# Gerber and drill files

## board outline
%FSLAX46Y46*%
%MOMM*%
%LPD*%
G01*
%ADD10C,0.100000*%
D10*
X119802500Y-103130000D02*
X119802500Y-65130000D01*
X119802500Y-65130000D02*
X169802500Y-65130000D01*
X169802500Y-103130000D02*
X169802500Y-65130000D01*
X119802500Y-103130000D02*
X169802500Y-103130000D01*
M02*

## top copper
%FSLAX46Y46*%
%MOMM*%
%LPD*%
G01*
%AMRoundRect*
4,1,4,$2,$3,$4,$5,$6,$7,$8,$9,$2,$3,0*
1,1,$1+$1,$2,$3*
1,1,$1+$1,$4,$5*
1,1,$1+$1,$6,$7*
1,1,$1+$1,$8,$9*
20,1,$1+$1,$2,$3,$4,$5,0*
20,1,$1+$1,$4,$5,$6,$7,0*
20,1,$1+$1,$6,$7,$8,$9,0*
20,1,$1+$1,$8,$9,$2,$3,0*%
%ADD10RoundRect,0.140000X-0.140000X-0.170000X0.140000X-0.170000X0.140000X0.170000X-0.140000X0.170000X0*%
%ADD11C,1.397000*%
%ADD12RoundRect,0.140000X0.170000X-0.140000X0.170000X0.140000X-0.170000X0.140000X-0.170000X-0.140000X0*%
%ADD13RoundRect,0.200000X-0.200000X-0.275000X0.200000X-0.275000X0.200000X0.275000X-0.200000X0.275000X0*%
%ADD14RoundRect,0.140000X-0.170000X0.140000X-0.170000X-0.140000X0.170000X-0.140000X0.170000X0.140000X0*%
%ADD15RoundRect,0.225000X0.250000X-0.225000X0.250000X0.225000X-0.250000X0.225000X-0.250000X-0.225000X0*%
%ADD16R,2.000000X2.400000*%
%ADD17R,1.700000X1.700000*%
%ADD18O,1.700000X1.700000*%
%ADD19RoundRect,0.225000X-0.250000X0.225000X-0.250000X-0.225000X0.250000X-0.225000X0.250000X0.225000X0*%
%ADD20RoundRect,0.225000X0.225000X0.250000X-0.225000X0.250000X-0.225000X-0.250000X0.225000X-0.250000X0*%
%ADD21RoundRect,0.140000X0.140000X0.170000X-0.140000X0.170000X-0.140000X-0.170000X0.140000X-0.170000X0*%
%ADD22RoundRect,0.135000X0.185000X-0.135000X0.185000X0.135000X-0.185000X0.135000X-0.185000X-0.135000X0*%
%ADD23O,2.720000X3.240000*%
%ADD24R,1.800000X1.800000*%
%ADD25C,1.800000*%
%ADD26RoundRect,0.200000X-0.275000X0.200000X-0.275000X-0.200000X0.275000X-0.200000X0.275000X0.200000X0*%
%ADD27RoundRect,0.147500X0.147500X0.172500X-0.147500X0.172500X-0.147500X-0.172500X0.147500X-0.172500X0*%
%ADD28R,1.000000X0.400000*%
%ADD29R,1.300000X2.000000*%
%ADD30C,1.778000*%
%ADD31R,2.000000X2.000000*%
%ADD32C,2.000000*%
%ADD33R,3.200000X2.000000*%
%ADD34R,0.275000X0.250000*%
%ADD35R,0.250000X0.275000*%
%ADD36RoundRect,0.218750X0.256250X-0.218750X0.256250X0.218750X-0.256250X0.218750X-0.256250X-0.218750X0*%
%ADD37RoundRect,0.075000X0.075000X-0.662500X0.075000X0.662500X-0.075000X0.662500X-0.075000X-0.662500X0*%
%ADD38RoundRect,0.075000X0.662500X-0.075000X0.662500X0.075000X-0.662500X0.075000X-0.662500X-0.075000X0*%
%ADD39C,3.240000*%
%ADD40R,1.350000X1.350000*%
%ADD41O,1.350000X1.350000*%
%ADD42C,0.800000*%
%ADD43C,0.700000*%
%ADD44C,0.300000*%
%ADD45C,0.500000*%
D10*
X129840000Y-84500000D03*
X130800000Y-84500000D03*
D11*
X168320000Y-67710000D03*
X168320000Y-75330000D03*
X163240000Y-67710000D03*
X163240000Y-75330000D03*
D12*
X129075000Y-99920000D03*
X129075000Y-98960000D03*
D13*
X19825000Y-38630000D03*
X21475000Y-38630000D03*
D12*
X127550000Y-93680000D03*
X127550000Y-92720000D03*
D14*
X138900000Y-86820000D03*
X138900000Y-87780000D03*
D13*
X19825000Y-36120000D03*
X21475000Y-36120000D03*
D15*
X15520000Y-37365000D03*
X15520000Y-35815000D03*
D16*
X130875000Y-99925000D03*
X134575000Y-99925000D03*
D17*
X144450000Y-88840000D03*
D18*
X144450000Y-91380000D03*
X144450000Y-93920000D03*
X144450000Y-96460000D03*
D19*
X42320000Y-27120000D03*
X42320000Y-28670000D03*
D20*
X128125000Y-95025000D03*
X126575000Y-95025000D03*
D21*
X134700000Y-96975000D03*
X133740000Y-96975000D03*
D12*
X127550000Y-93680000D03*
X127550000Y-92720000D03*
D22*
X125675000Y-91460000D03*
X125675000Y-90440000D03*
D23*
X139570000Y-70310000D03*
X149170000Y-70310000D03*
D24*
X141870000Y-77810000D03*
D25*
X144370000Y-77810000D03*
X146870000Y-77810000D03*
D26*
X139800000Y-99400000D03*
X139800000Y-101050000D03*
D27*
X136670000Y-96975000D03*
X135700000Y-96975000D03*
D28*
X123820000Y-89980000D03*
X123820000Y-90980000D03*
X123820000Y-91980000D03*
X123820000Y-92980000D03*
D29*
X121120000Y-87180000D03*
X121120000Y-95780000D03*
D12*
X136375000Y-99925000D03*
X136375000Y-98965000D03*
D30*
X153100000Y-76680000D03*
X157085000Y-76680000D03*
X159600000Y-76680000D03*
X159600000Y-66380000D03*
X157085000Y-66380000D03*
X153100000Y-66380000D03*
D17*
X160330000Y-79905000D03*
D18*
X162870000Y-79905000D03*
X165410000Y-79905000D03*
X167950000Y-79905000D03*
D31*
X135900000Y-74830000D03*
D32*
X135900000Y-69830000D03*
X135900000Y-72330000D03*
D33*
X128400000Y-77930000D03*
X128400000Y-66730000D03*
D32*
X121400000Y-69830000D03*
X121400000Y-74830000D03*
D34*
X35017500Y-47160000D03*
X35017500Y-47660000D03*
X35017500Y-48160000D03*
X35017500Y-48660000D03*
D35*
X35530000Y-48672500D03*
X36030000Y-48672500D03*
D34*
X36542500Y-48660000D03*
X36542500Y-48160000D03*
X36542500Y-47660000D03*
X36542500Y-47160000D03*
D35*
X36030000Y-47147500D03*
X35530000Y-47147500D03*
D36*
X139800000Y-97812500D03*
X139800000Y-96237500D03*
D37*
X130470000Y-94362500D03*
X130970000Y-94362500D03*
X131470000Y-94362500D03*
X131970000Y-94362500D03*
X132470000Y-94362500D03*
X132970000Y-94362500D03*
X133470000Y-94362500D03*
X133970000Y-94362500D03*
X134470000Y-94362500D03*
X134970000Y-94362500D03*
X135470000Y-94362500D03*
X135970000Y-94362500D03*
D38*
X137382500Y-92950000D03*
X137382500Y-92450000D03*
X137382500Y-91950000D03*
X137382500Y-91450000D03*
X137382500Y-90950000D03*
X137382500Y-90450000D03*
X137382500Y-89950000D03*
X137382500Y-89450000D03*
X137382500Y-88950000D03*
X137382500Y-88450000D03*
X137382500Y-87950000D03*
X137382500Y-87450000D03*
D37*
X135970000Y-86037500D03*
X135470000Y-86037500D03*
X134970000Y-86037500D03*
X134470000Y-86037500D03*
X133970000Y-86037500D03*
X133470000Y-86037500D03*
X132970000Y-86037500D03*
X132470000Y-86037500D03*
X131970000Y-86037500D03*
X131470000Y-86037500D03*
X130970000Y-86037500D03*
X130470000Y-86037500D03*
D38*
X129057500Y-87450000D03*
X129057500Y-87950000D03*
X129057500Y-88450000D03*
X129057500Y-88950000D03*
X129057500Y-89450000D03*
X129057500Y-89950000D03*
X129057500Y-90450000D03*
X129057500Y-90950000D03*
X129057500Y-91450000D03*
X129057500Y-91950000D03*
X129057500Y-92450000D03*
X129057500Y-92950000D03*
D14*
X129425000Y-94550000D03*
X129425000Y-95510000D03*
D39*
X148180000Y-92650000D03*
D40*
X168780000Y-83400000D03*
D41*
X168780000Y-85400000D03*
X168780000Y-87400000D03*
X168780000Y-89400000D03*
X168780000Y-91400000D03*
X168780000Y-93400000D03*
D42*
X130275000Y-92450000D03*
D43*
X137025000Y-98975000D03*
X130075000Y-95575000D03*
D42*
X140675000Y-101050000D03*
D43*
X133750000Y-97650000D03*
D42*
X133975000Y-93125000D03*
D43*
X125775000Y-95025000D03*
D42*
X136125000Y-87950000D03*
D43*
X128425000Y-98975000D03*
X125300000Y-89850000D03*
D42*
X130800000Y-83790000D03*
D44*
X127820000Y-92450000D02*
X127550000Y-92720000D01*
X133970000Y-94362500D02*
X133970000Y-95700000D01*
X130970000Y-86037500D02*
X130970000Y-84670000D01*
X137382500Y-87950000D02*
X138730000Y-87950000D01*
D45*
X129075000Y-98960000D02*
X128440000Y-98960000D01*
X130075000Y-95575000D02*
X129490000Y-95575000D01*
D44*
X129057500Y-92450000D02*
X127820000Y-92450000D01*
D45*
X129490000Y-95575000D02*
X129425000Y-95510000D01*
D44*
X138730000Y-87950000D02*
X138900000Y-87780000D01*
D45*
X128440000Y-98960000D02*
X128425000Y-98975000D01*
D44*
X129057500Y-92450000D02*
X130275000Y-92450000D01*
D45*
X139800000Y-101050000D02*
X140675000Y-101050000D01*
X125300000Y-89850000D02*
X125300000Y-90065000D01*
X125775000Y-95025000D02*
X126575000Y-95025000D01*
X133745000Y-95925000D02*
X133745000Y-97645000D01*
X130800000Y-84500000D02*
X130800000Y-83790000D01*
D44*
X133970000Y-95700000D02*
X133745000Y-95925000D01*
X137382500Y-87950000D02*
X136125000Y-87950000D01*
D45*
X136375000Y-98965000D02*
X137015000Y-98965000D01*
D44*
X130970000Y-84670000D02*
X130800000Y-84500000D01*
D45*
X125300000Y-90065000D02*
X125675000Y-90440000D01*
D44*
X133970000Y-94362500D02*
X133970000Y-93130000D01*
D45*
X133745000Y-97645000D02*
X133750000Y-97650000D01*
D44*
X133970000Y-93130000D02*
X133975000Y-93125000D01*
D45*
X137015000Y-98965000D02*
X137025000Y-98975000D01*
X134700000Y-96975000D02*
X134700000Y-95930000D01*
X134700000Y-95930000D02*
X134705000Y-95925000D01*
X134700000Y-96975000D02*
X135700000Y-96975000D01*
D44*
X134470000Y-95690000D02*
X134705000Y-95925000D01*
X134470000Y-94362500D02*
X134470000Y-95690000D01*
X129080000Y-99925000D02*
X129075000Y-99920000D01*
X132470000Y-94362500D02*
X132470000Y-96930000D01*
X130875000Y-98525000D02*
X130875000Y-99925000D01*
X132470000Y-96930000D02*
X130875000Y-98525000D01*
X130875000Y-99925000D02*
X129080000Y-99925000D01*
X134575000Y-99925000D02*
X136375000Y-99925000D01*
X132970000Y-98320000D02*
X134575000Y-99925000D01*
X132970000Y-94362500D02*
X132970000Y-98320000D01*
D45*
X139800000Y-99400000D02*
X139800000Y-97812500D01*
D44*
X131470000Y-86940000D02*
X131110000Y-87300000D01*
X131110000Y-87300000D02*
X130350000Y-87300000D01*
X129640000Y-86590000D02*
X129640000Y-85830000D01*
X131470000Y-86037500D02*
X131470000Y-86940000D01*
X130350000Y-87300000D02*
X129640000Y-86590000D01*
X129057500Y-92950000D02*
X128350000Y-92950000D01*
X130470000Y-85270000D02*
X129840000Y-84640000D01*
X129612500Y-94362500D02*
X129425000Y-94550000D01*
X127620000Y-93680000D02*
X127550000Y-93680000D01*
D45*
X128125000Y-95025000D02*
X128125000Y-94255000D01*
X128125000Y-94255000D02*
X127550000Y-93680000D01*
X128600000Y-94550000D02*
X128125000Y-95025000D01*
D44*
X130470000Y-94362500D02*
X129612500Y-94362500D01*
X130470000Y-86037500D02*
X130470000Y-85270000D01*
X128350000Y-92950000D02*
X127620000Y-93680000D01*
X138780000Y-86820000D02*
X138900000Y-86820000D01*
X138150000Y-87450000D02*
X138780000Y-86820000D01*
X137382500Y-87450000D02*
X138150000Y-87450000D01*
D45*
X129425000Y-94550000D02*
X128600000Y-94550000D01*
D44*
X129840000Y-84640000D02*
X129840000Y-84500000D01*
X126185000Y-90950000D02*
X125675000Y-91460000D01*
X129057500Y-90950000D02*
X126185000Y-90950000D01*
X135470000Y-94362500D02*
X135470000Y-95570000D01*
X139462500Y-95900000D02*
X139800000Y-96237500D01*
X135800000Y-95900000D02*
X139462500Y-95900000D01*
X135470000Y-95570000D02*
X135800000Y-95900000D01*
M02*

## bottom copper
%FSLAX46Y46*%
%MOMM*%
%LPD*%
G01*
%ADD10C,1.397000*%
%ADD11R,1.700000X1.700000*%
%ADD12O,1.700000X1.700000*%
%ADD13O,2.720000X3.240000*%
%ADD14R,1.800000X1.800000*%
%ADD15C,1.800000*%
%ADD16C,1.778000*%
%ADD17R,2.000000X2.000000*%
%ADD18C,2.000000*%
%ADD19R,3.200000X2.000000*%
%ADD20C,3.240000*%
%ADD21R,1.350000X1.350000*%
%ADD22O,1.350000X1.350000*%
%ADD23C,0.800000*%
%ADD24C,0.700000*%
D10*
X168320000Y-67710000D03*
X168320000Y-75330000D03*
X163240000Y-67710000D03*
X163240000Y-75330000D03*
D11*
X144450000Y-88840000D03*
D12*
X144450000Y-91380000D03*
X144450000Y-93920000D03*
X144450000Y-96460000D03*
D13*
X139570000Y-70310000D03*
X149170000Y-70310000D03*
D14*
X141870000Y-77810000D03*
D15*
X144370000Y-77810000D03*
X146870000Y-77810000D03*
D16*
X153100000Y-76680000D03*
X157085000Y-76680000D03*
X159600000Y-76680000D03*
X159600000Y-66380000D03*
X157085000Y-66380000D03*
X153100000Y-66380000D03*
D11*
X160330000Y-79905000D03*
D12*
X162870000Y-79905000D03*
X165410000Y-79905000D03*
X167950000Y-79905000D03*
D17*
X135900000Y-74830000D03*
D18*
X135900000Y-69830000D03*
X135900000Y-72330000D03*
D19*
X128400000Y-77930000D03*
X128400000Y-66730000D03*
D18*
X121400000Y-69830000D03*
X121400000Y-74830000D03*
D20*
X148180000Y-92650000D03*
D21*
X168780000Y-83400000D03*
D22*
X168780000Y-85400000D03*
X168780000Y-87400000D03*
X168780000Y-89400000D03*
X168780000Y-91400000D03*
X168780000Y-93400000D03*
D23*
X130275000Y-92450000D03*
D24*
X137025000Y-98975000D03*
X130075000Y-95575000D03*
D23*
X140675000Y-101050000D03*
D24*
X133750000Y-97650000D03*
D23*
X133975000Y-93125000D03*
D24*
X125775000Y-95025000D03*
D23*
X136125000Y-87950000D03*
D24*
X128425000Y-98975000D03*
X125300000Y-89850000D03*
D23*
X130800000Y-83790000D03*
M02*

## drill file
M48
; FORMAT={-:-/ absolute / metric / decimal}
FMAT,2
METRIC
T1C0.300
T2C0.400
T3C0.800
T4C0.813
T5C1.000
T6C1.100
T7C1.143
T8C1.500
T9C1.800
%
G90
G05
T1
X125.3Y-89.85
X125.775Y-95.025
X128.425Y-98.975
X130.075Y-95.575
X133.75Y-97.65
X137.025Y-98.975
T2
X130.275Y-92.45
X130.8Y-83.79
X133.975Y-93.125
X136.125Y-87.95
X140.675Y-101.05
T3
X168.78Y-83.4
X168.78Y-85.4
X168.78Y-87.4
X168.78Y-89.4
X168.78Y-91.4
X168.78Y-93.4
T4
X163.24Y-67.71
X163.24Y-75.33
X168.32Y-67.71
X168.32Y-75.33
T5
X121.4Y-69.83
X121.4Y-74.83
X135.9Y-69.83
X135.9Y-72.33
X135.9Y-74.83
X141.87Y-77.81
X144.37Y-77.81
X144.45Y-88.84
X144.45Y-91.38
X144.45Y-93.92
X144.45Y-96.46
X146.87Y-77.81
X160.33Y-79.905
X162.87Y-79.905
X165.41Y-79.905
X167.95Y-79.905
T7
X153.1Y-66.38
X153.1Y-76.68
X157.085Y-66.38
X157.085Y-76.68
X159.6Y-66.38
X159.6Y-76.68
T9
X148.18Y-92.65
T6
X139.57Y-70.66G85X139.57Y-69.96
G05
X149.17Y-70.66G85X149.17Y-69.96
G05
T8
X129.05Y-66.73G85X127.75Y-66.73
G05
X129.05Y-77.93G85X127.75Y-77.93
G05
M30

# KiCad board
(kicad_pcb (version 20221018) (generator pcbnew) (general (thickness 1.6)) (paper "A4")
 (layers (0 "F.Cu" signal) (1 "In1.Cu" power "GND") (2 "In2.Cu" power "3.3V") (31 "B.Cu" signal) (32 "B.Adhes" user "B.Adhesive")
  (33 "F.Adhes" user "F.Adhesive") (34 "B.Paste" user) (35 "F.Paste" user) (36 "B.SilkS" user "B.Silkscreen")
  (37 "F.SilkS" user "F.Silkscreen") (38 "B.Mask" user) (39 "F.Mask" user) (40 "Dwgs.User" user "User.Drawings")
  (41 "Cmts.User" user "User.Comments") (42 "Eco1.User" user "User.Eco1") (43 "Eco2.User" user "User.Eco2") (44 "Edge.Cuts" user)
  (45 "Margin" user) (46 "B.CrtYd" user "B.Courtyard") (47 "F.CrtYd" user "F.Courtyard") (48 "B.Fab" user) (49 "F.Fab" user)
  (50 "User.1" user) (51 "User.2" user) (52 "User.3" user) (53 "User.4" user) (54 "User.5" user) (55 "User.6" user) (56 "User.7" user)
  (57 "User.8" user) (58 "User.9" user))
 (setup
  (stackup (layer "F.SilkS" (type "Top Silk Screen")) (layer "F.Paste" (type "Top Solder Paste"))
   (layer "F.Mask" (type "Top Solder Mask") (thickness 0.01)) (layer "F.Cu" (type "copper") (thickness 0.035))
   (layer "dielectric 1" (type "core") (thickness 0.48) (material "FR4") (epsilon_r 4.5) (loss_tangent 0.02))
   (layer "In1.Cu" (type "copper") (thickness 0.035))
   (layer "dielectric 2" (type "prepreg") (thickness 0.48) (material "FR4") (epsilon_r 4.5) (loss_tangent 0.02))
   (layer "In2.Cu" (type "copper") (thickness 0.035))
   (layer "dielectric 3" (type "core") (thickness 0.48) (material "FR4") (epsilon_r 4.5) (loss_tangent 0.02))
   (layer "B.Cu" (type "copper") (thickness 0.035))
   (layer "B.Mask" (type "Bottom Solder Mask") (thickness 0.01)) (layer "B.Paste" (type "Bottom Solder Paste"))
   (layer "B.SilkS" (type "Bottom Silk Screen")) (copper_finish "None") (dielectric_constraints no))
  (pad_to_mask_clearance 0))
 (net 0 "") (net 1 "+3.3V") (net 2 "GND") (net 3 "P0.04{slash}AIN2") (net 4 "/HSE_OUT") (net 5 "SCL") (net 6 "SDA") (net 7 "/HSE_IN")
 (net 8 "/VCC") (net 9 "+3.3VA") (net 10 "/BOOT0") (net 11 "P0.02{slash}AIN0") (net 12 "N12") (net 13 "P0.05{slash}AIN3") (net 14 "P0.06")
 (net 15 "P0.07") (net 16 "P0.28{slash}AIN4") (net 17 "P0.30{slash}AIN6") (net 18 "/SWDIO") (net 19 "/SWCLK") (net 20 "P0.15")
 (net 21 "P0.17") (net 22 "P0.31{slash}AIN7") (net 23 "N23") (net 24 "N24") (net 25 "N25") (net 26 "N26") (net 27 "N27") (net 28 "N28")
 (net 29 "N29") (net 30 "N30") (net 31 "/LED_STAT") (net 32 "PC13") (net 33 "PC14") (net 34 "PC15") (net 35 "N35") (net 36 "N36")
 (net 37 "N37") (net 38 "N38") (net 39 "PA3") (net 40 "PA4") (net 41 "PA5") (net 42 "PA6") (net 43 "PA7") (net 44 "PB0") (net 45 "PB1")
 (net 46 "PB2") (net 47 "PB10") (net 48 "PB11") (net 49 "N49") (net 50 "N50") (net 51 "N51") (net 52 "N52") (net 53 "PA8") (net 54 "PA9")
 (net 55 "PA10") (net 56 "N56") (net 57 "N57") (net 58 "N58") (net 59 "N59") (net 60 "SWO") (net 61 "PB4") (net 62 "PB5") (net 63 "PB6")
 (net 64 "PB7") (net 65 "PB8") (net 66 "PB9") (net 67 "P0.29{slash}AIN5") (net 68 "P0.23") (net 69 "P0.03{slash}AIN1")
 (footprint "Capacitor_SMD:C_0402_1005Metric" (layer "F.Cu") (at 130.32 84.5)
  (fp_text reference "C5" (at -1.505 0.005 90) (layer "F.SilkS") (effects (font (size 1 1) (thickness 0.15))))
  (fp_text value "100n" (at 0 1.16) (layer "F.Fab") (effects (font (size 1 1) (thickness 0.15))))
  (pad "1" smd roundrect (at -0.48 0) (size 0.56 0.62) (layers "F.Cu" "F.Paste" "F.Mask") (roundrect_rratio 0.25) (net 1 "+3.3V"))
  (pad "2" smd roundrect (at 0.48 0) (size 0.56 0.62) (layers "F.Cu" "F.Paste" "F.Mask") (roundrect_rratio 0.25) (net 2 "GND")))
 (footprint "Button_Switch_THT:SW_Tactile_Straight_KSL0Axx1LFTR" (layer "F.Cu") (at 168.32 67.71 -90)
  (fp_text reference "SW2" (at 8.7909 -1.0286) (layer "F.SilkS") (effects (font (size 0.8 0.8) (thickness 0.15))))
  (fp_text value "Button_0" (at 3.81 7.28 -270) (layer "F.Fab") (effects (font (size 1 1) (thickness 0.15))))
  (pad "1" thru_hole circle (at 0 0 270) (size 1.397 1.397) (drill 0.8128) (layers "*.Cu" "*.Mask") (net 2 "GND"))
  (pad "1" thru_hole circle (at 7.62 0 270) (size 1.397 1.397) (drill 0.8128) (layers "*.Cu" "*.Mask") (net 2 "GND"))
  (pad "2" thru_hole circle (at 0 5.08 270) (size 1.397 1.397) (drill 0.8128) (layers "*.Cu" "*.Mask") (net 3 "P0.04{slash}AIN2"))
  (pad "2" thru_hole circle (at 7.62 5.08 270) (size 1.397 1.397) (drill 0.8128) (layers "*.Cu" "*.Mask") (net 3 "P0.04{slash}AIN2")))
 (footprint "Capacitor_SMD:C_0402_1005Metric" (layer "F.Cu") (at 129.075 99.44 90)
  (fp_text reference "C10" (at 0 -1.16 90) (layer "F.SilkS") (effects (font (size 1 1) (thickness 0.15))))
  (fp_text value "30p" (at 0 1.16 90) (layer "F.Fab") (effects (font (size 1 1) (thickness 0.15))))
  (pad "1" smd roundrect (at -0.48 0 90) (size 0.56 0.62) (layers "F.Cu" "F.Paste" "F.Mask") (roundrect_rratio 0.25) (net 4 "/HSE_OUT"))
  (pad "2" smd roundrect (at 0.48 0 90) (size 0.56 0.62) (layers "F.Cu" "F.Paste" "F.Mask") (roundrect_rratio 0.25) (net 2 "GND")))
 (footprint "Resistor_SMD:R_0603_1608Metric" (layer "F.Cu") (at 20.65 38.63)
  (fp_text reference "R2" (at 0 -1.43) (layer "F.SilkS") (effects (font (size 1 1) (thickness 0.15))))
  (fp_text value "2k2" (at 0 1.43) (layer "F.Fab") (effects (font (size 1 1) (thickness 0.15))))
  (pad "1" smd roundrect (at -0.825 0) (size 0.8 0.95) (layers "F.Cu" "F.Paste" "F.Mask") (roundrect_rratio 0.25) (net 1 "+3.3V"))
  (pad "2" smd roundrect (at 0.825 0) (size 0.8 0.95) (layers "F.Cu" "F.Paste" "F.Mask") (roundrect_rratio 0.25) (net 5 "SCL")))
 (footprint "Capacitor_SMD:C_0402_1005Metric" (layer "F.Cu") (at 127.55 93.2 90)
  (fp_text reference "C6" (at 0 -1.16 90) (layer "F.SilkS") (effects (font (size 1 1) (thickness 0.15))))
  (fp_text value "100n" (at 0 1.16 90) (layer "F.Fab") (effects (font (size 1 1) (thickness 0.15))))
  (pad "1" smd roundrect (at -0.48 0 90) (size 0.56 0.62) (layers "F.Cu" "F.Paste" "F.Mask") (roundrect_rratio 0.25) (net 1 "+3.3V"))
  (pad "2" smd roundrect (at 0.48 0 90) (size 0.56 0.62) (layers "F.Cu" "F.Paste" "F.Mask") (roundrect_rratio 0.25) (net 2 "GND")))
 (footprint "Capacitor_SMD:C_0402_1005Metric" (layer "F.Cu") (at 138.9 87.3 -90)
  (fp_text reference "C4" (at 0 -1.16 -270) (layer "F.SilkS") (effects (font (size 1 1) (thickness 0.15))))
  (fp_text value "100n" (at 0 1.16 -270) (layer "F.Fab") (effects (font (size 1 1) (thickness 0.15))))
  (pad "1" smd roundrect (at -0.48 0 270) (size 0.56 0.62) (layers "F.Cu" "F.Paste" "F.Mask") (roundrect_rratio 0.25) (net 1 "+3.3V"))
  (pad "2" smd roundrect (at 0.48 0 270) (size 0.56 0.62) (layers "F.Cu" "F.Paste" "F.Mask") (roundrect_rratio 0.25) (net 2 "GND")))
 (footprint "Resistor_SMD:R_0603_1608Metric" (layer "F.Cu") (at 20.65 36.12)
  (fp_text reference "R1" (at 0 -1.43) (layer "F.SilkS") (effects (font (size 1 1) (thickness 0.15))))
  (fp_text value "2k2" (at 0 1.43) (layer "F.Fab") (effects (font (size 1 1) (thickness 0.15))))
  (pad "1" smd roundrect (at -0.825 0) (size 0.8 0.95) (layers "F.Cu" "F.Paste" "F.Mask") (roundrect_rratio 0.25) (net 1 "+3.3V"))
  (pad "2" smd roundrect (at 0.825 0) (size 0.8 0.95) (layers "F.Cu" "F.Paste" "F.Mask") (roundrect_rratio 0.25) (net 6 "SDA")))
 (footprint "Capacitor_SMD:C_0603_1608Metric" (layer "F.Cu") (at 15.52 36.59 90)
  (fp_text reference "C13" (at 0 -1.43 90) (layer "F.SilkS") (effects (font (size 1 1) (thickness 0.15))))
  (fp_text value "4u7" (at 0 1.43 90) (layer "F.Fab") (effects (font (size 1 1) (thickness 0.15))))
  (pad "1" smd roundrect (at -0.775 0 90) (size 0.9 0.95) (layers "F.Cu" "F.Paste" "F.Mask") (roundrect_rratio 0.25) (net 1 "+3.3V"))
  (pad "2" smd roundrect (at 0.775 0 90) (size 0.9 0.95) (layers "F.Cu" "F.Paste" "F.Mask") (roundrect_rratio 0.25) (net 2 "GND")))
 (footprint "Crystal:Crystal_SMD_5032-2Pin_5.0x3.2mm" (layer "F.Cu") (at 132.725 99.925)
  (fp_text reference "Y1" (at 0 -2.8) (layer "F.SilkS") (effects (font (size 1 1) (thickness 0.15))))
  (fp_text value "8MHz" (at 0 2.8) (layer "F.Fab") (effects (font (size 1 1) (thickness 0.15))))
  (pad "1" smd rect (at -1.85 0) (size 2 2.4) (layers "F.Cu" "F.Paste" "F.Mask") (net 4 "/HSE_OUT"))
  (pad "2" smd rect (at 1.85 0) (size 2 2.4) (layers "F.Cu" "F.Paste" "F.Mask") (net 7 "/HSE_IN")))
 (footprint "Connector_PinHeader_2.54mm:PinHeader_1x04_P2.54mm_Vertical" (layer "F.Cu") (at 144.45 88.84)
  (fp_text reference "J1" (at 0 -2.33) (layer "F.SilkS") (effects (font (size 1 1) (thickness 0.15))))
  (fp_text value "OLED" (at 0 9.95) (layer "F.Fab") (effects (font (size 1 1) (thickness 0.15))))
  (pad "1" thru_hole rect (at 0 0) (size 1.7 1.7) (drill 1) (layers "*.Cu" "*.Mask") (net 2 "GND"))
  (pad "2" thru_hole oval (at 0 2.54) (size 1.7 1.7) (drill 1) (layers "*.Cu" "*.Mask") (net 1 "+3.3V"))
  (pad "3" thru_hole oval (at 0 5.08) (size 1.7 1.7) (drill 1) (layers "*.Cu" "*.Mask") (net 5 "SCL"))
  (pad "4" thru_hole oval (at 0 7.62) (size 1.7 1.7) (drill 1) (layers "*.Cu" "*.Mask") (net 6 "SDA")))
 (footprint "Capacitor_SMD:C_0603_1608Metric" (layer "F.Cu") (at 42.32 27.895 -90)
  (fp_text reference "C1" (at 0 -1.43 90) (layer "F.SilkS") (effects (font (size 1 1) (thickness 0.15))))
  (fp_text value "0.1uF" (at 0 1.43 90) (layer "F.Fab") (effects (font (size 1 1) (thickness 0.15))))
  (pad "1" smd roundrect (at -0.775 0 270) (size 0.9 0.95) (layers "F.Cu" "F.Paste" "F.Mask") (roundrect_rratio 0.25) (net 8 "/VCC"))
  (pad "2" smd roundrect (at 0.775 0 270) (size 0.9 0.95) (layers "F.Cu" "F.Paste" "F.Mask") (roundrect_rratio 0.25) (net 2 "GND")))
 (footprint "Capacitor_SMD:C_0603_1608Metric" (layer "F.Cu") (at 127.35 95.025 180)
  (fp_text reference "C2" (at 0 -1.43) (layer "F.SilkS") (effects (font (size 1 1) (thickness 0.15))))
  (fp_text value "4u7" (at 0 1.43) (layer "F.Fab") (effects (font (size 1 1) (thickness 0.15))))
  (pad "1" smd roundrect (at -0.775 0 180) (size 0.9 0.95) (layers "F.Cu" "F.Paste" "F.Mask") (roundrect_rratio 0.25) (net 1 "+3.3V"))
  (pad "2" smd roundrect (at 0.775 0 180) (size 0.9 0.95) (layers "F.Cu" "F.Paste" "F.Mask") (roundrect_rratio 0.25) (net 2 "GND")))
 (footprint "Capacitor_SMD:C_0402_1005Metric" (layer "F.Cu") (at 134.22 96.975 180)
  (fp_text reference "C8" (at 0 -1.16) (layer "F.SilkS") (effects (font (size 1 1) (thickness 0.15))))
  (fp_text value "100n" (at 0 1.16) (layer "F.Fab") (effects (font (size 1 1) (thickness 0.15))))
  (pad "1" smd roundrect (at -0.48 0 180) (size 0.56 0.62) (layers "F.Cu" "F.Paste" "F.Mask") (roundrect_rratio 0.25) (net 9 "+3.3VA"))
  (pad "2" smd roundrect (at 0.48 0 180) (size 0.56 0.62) (layers "F.Cu" "F.Paste" "F.Mask") (roundrect_rratio 0.25) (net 2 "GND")))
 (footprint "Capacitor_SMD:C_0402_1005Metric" (layer "F.Cu") (at 127.55 93.2 90)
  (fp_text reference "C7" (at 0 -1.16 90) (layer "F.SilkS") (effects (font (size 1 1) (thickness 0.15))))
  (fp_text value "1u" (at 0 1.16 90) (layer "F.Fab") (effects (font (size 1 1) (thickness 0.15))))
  (pad "1" smd roundrect (at -0.48 0 90) (size 0.56 0.62) (layers "F.Cu" "F.Paste" "F.Mask") (roundrect_rratio 0.25) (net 9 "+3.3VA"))
  (pad "2" smd roundrect (at 0.48 0 90) (size 0.56 0.62) (layers "F.Cu" "F.Paste" "F.Mask") (roundrect_rratio 0.25) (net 2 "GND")))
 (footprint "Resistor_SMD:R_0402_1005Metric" (layer "F.Cu") (at 125.675 90.95 90)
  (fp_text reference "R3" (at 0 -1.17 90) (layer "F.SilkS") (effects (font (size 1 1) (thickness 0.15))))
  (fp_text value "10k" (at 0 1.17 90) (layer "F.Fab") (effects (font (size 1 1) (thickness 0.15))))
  (pad "1" smd roundrect (at -0.51 0 90) (size 0.54 0.64) (layers "F.Cu" "F.Paste" "F.Mask") (roundrect_rratio 0.25) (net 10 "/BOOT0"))
  (pad "2" smd roundrect (at 0.51 0 90) (size 0.54 0.64) (layers "F.Cu" "F.Paste" "F.Mask") (roundrect_rratio 0.25) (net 2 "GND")))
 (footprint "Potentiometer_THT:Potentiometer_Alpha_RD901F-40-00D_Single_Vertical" (layer "F.Cu") (at 141.87 77.81 90)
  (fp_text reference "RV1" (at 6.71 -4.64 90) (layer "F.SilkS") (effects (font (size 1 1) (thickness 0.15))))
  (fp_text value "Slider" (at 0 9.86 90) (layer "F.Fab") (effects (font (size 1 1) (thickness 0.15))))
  (pad "" thru_hole oval (at 7.5 -2.3 180) (size 2.72 3.24) (drill oval 1.1 1.8) (layers "*.Cu" "*.Mask"))
  (pad "" thru_hole oval (at 7.5 7.3 180) (size 2.72 3.24) (drill oval 1.1 1.8) (layers "*.Cu" "*.Mask"))
  (pad "1" thru_hole rect (at 0 0 180) (size 1.8 1.8) (drill 1) (layers "*.Cu" "*.Mask") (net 1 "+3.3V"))
  (pad "2" thru_hole circle (at 0 2.5 180) (size 1.8 1.8) (drill 1) (layers "*.Cu" "*.Mask") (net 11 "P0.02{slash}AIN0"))
  (pad "3" thru_hole circle (at 0 5 180) (size 1.8 1.8) (drill 1) (layers "*.Cu" "*.Mask") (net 2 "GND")))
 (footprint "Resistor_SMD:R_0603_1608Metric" (layer "F.Cu") (at 139.8 100.225 -90)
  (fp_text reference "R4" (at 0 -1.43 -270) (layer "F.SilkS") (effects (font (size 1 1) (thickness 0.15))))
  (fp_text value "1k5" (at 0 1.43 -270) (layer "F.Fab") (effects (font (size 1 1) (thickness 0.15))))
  (pad "1" smd roundrect (at -0.825 0 270) (size 0.8 0.95) (layers "F.Cu" "F.Paste" "F.Mask") (roundrect_rratio 0.25) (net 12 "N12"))
  (pad "2" smd roundrect (at 0.825 0 270) (size 0.8 0.95) (layers "F.Cu" "F.Paste" "F.Mask") (roundrect_rratio 0.25) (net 2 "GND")))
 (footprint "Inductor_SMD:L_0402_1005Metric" (layer "F.Cu") (at 136.185 96.975 180)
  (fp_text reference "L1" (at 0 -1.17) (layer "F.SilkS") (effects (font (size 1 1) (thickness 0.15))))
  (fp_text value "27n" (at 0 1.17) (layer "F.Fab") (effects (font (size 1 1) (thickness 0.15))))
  (pad "1" smd roundrect (at -0.485 0 180) (size 0.59 0.64) (layers "F.Cu" "F.Paste" "F.Mask") (roundrect_rratio 0.25) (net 1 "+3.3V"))
  (pad "2" smd roundrect (at 0.485 0 180) (size 0.59 0.64) (layers "F.Cu" "F.Paste" "F.Mask") (roundrect_rratio 0.25) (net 9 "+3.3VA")))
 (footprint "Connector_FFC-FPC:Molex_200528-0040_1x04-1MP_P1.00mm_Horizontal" (layer "F.Cu") (at 122.91 91.48 -90)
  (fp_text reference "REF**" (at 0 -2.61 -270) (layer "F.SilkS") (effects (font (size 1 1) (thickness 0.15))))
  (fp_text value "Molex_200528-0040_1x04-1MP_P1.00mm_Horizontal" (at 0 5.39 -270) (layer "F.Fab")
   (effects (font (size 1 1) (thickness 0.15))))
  (pad "1" smd rect (at -1.5 -0.91 270) (size 0.4 1) (layers "F.Cu" "F.Paste" "F.Mask"))
  (pad "2" smd rect (at -0.5 -0.91 270) (size 0.4 1) (layers "F.Cu" "F.Paste" "F.Mask"))
  (pad "3" smd rect (at 0.5 -0.91 270) (size 0.4 1) (layers "F.Cu" "F.Paste" "F.Mask"))
  (pad "4" smd rect (at 1.5 -0.91 270) (size 0.4 1) (layers "F.Cu" "F.Paste" "F.Mask"))
  (pad "MP" smd rect (at -4.3 1.79 270) (size 2 1.3) (layers "F.Cu" "F.Paste" "F.Mask"))
  (pad "MP" smd rect (at 4.3 1.79 270) (size 2 1.3) (layers "F.Cu" "F.Paste" "F.Mask")))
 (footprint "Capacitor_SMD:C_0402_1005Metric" (layer "F.Cu") (at 136.375 99.445 90)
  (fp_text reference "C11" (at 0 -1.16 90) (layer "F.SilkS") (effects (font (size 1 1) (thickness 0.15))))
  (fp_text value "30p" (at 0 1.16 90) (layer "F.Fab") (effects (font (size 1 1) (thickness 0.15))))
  (pad "1" smd roundrect (at -0.48 0 90) (size 0.56 0.62) (layers "F.Cu" "F.Paste" "F.Mask") (roundrect_rratio 0.25) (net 7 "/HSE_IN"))
  (pad "2" smd roundrect (at 0.48 0 90) (size 0.56 0.62) (layers "F.Cu" "F.Paste" "F.Mask") (roundrect_rratio 0.25) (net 2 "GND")))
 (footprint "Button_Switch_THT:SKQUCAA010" (layer "F.Cu") (at 156.635 71.52 90)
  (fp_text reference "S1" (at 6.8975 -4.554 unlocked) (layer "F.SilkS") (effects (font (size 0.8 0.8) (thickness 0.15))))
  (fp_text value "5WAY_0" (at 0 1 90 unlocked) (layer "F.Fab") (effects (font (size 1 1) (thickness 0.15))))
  (pad "1" thru_hole circle (at -5.16 -3.535 180) (size 1.778 1.778) (drill 1.143) (layers "*.Cu" "*.Mask") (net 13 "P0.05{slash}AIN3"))
  (pad "2" thru_hole circle (at -5.16 0.45 180) (size 1.778 1.778) (drill 1.143) (layers "*.Cu" "*.Mask") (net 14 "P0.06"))
  (pad "3" thru_hole circle (at -5.16 2.965 180) (size 1.778 1.778) (drill 1.143) (layers "*.Cu" "*.Mask") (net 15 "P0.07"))
  (pad "4" thru_hole circle (at 5.14 2.965 180) (size 1.778 1.778) (drill 1.143) (layers "*.Cu" "*.Mask") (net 2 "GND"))
  (pad "5" thru_hole circle (at 5.14 0.45 180) (size 1.778 1.778) (drill 1.143) (layers "*.Cu" "*.Mask") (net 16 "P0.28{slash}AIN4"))
  (pad "6" thru_hole circle (at 5.14 -3.535 180) (size 1.778 1.778) (drill 1.143) (layers "*.Cu" "*.Mask") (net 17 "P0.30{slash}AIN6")))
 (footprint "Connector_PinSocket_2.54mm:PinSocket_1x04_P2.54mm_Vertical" (layer "F.Cu") (at 160.33 79.905 90)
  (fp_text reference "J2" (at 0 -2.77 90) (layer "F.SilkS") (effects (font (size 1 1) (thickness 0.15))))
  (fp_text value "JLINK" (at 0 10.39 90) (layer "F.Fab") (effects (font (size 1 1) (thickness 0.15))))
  (pad "1" thru_hole rect (at 0 0 90) (size 1.7 1.7) (drill 1) (layers "*.Cu" "*.Mask") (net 8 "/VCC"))
  (pad "2" thru_hole oval (at 0 2.54 90) (size 1.7 1.7) (drill 1) (layers "*.Cu" "*.Mask") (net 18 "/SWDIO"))
  (pad "3" thru_hole oval (at 0 5.08 90) (size 1.7 1.7) (drill 1) (layers "*.Cu" "*.Mask") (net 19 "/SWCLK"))
  (pad "4" thru_hole oval (at 0 7.62 90) (size 1.7 1.7) (drill 1) (layers "*.Cu" "*.Mask") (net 2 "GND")))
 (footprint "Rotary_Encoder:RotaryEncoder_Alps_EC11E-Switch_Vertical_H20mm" (layer "F.Cu") (at 135.9 74.83 180)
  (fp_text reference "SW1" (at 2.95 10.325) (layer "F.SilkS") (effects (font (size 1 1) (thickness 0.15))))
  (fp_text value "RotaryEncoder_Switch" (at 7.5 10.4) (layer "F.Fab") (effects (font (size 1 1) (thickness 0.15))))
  (pad "A" thru_hole rect (at 0 0 180) (size 2 2) (drill 1) (layers "*.Cu" "*.Mask") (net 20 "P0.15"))
  (pad "B" thru_hole circle (at 0 5 180) (size 2 2) (drill 1) (layers "*.Cu" "*.Mask") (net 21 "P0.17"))
  (pad "C" thru_hole circle (at 0 2.5 180) (size 2 2) (drill 1) (layers "*.Cu" "*.Mask") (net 2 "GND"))
  (pad "MP" thru_hole rect (at 7.5 -3.1 180) (size 3.2 2) (drill oval 2.8 1.5) (layers "*.Cu" "*.Mask"))
  (pad "MP" thru_hole rect (at 7.5 8.1 180) (size 3.2 2) (drill oval 2.8 1.5) (layers "*.Cu" "*.Mask"))
  (pad "S1" thru_hole circle (at 14.5 5 180) (size 2 2) (drill 1) (layers "*.Cu" "*.Mask") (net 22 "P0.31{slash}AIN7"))
  (pad "S2" thru_hole circle (at 14.5 0 180) (size 2 2) (drill 1) (layers "*.Cu" "*.Mask") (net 2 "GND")))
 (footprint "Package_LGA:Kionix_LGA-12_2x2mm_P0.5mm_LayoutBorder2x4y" (layer "F.Cu") (at 35.78 47.91)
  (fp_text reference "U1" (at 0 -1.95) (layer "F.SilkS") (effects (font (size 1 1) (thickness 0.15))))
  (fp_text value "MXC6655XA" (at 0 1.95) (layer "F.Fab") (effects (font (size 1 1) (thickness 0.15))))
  (pad "1" smd rect (at -0.7625 -0.75) (size 0.275 0.25) (layers "F.Cu" "F.Paste" "F.Mask") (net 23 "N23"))
  (pad "2" smd rect (at -0.7625 -0.25) (size 0.275 0.25) (layers "F.Cu" "F.Paste" "F.Mask") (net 6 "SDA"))
  (pad "3" smd rect (at -0.7625 0.25) (size 0.275 0.25) (layers "F.Cu" "F.Paste" "F.Mask") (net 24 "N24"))
  (pad "4" smd rect (at -0.7625 0.75) (size 0.275 0.25) (layers "F.Cu" "F.Paste" "F.Mask") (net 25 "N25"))
  (pad "5" smd rect (at -0.25 0.7625) (size 0.25 0.275) (layers "F.Cu" "F.Paste" "F.Mask") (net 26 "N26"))
  (pad "6" smd rect (at 0.25 0.7625) (size 0.25 0.275) (layers "F.Cu" "F.Paste" "F.Mask") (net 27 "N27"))
  (pad "7" smd rect (at 0.7625 0.75) (size 0.275 0.25) (layers "F.Cu" "F.Paste" "F.Mask") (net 1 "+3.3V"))
  (pad "8" smd rect (at 0.7625 0.25) (size 0.275 0.25) (layers "F.Cu" "F.Paste" "F.Mask") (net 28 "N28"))
  (pad "9" smd rect (at 0.7625 -0.25) (size 0.275 0.25) (layers "F.Cu" "F.Paste" "F.Mask") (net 2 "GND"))
  (pad "10" smd rect (at 0.7625 -0.75) (size 0.275 0.25) (layers "F.Cu" "F.Paste" "F.Mask") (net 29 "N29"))
  (pad "11" smd rect (at 0.25 -0.7625) (size 0.25 0.275) (layers "F.Cu" "F.Paste" "F.Mask") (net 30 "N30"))
  (pad "12" smd rect (at -0.25 -0.7625) (size 0.25 0.275) (layers "F.Cu" "F.Paste" "F.Mask") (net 5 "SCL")))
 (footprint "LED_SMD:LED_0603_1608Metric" (layer "F.Cu") (at 139.8 97.025 90)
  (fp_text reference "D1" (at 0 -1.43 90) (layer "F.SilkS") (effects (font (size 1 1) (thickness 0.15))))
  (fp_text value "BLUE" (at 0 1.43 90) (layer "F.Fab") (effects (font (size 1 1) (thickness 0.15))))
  (pad "1" smd roundrect (at -0.7875 0 90) (size 0.875 0.95) (layers "F.Cu" "F.Paste" "F.Mask") (roundrect_rratio 0.25) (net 12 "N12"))
  (pad "2" smd roundrect (at 0.7875 0 90) (size 0.875 0.95) (layers "F.Cu" "F.Paste" "F.Mask") (roundrect_rratio 0.25) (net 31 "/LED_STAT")))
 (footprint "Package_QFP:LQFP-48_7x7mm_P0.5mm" (layer "F.Cu") (at 133.22 90.2 90)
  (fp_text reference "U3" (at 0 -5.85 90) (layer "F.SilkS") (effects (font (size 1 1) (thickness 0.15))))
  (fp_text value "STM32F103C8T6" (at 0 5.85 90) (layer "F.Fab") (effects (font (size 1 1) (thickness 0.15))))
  (pad "1" smd roundrect (at -4.1625 -2.75 90) (size 1.475 0.3) (layers "F.Cu" "F.Paste" "F.Mask") (roundrect_rratio 0.25) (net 1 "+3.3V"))
  (pad "2" smd roundrect (at -4.1625 -2.25 90) (size 1.475 0.3) (layers "F.Cu" "F.Paste" "F.Mask") (roundrect_rratio 0.25) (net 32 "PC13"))
  (pad "3" smd roundrect (at -4.1625 -1.75 90) (size 1.475 0.3) (layers "F.Cu" "F.Paste" "F.Mask") (roundrect_rratio 0.25) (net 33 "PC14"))
  (pad "4" smd roundrect (at -4.1625 -1.25 90) (size 1.475 0.3) (layers "F.Cu" "F.Paste" "F.Mask") (roundrect_rratio 0.25) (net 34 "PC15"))
  (pad "5" smd roundrect (at -4.1625 -0.75 90) (size 1.475 0.3) (layers "F.Cu" "F.Paste" "F.Mask") (roundrect_rratio 0.25)
   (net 4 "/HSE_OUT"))
  (pad "6" smd roundrect (at -4.1625 -0.25 90) (size 1.475 0.3) (layers "F.Cu" "F.Paste" "F.Mask") (roundrect_rratio 0.25) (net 7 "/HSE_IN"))
  (pad "7" smd roundrect (at -4.1625 0.25 90) (size 1.475 0.3) (layers "F.Cu" "F.Paste" "F.Mask") (roundrect_rratio 0.25) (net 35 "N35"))
  (pad "8" smd roundrect (at -4.1625 0.75 90) (size 1.475 0.3) (layers "F.Cu" "F.Paste" "F.Mask") (roundrect_rratio 0.25) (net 2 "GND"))
  (pad "9" smd roundrect (at -4.1625 1.25 90) (size 1.475 0.3) (layers "F.Cu" "F.Paste" "F.Mask") (roundrect_rratio 0.25) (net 9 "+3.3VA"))
  (pad "10" smd roundrect (at -4.1625 1.75 90) (size 1.475 0.3) (layers "F.Cu" "F.Paste" "F.Mask") (roundrect_rratio 0.25) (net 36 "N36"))
  (pad "11" smd roundrect (at -4.1625 2.25 90) (size 1.475 0.3) (layers "F.Cu" "F.Paste" "F.Mask") (roundrect_rratio 0.25) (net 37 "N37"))
  (pad "12" smd roundrect (at -4.1625 2.75 90) (size 1.475 0.3) (layers "F.Cu" "F.Paste" "F.Mask") (roundrect_rratio 0.25) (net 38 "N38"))
  (pad "13" smd roundrect (at -2.75 4.1625 90) (size 0.3 1.475) (layers "F.Cu" "F.Paste" "F.Mask") (roundrect_rratio 0.25) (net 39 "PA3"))
  (pad "14" smd roundrect (at -2.25 4.1625 90) (size 0.3 1.475) (layers "F.Cu" "F.Paste" "F.Mask") (roundrect_rratio 0.25) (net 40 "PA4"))
  (pad "15" smd roundrect (at -1.75 4.1625 90) (size 0.3 1.475) (layers "F.Cu" "F.Paste" "F.Mask") (roundrect_rratio 0.25) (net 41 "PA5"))
  (pad "16" smd roundrect (at -1.25 4.1625 90) (size 0.3 1.475) (layers "F.Cu" "F.Paste" "F.Mask") (roundrect_rratio 0.25) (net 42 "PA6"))
  (pad "17" smd roundrect (at -0.75 4.1625 90) (size 0.3 1.475) (layers "F.Cu" "F.Paste" "F.Mask") (roundrect_rratio 0.25) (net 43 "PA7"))
  (pad "18" smd roundrect (at -0.25 4.1625 90) (size 0.3 1.475) (layers "F.Cu" "F.Paste" "F.Mask") (roundrect_rratio 0.25) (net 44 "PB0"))
  (pad "19" smd roundrect (at 0.25 4.1625 90) (size 0.3 1.475) (layers "F.Cu" "F.Paste" "F.Mask") (roundrect_rratio 0.25) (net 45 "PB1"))
  (pad "20" smd roundrect (at 0.75 4.1625 90) (size 0.3 1.475) (layers "F.Cu" "F.Paste" "F.Mask") (roundrect_rratio 0.25) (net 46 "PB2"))
  (pad "21" smd roundrect (at 1.25 4.1625 90) (size 0.3 1.475) (layers "F.Cu" "F.Paste" "F.Mask") (roundrect_rratio 0.25) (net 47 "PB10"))
  (pad "22" smd roundrect (at 1.75 4.1625 90) (size 0.3 1.475) (layers "F.Cu" "F.Paste" "F.Mask") (roundrect_rratio 0.25) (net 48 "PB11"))
  (pad "23" smd roundrect (at 2.25 4.1625 90) (size 0.3 1.475) (layers "F.Cu" "F.Paste" "F.Mask") (roundrect_rratio 0.25) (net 2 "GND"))
  (pad "24" smd roundrect (at 2.75 4.1625 90) (size 0.3 1.475) (layers "F.Cu" "F.Paste" "F.Mask") (roundrect_rratio 0.25) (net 1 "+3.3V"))
  (pad "25" smd roundrect (at 4.1625 2.75 90) (size 1.475 0.3) (layers "F.Cu" "F.Paste" "F.Mask") (roundrect_rratio 0.25) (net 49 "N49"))
  (pad "26" smd roundrect (at 4.1625 2.25 90) (size 1.475 0.3) (layers "F.Cu" "F.Paste" "F.Mask") (roundrect_rratio 0.25) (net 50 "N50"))
  (pad "27" smd roundrect (at 4.1625 1.75 90) (size 1.475 0.3) (layers "F.Cu" "F.Paste" "F.Mask") (roundrect_rratio 0.25) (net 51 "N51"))
  (pad "28" smd roundrect (at 4.1625 1.25 90) (size 1.475 0.3) (layers "F.Cu" "F.Paste" "F.Mask") (roundrect_rratio 0.25) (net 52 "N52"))
  (pad "29" smd roundrect (at 4.1625 0.75 90) (size 1.475 0.3) (layers "F.Cu" "F.Paste" "F.Mask") (roundrect_rratio 0.25) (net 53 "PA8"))
  (pad "30" smd roundrect (at 4.1625 0.25 90) (size 1.475 0.3) (layers "F.Cu" "F.Paste" "F.Mask") (roundrect_rratio 0.25) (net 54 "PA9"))
  (pad "31" smd roundrect (at 4.1625 -0.25 90) (size 1.475 0.3) (layers "F.Cu" "F.Paste" "F.Mask") (roundrect_rratio 0.25) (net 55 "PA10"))
  (pad "32" smd roundrect (at 4.1625 -0.75 90) (size 1.475 0.3) (layers "F.Cu" "F.Paste" "F.Mask") (roundrect_rratio 0.25) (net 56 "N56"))
  (pad "33" smd roundrect (at 4.1625 -1.25 90) (size 1.475 0.3) (layers "F.Cu" "F.Paste" "F.Mask") (roundrect_rratio 0.25) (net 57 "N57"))
  (pad "34" smd roundrect (at 4.1625 -1.75 90) (size 1.475 0.3) (layers "F.Cu" "F.Paste" "F.Mask") (roundrect_rratio 0.25)
   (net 31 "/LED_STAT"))
  (pad "35" smd roundrect (at 4.1625 -2.25 90) (size 1.475 0.3) (layers "F.Cu" "F.Paste" "F.Mask") (roundrect_rratio 0.25) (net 2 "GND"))
  (pad "36" smd roundrect (at 4.1625 -2.75 90) (size 1.475 0.3) (layers "F.Cu" "F.Paste" "F.Mask") (roundrect_rratio 0.25) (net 1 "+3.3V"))
  (pad "37" smd roundrect (at 2.75 -4.1625 90) (size 0.3 1.475) (layers "F.Cu" "F.Paste" "F.Mask") (roundrect_rratio 0.25) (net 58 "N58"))
  (pad "38" smd roundrect (at 2.25 -4.1625 90) (size 0.3 1.475) (layers "F.Cu" "F.Paste" "F.Mask") (roundrect_rratio 0.25) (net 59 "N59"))
  (pad "39" smd roundrect (at 1.75 -4.1625 90) (size 0.3 1.475) (layers "F.Cu" "F.Paste" "F.Mask") (roundrect_rratio 0.25) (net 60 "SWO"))
  (pad "40" smd roundrect (at 1.25 -4.1625 90) (size 0.3 1.475) (layers "F.Cu" "F.Paste" "F.Mask") (roundrect_rratio 0.25) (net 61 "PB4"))
  (pad "41" smd roundrect (at 0.75 -4.1625 90) (size 0.3 1.475) (layers "F.Cu" "F.Paste" "F.Mask") (roundrect_rratio 0.25) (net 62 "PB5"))
  (pad "42" smd roundrect (at 0.25 -4.1625 90) (size 0.3 1.475) (layers "F.Cu" "F.Paste" "F.Mask") (roundrect_rratio 0.25) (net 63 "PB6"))
  (pad "43" smd roundrect (at -0.25 -4.1625 90) (size 0.3 1.475) (layers "F.Cu" "F.Paste" "F.Mask") (roundrect_rratio 0.25) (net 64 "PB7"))
  (pad "44" smd roundrect (at -0.75 -4.1625 90) (size 0.3 1.475) (layers "F.Cu" "F.Paste" "F.Mask") (roundrect_rratio 0.25)
   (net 10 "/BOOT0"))
  (pad "45" smd roundrect (at -1.25 -4.1625 90) (size 0.3 1.475) (layers "F.Cu" "F.Paste" "F.Mask") (roundrect_rratio 0.25) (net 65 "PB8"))
  (pad "46" smd roundrect (at -1.75 -4.1625 90) (size 0.3 1.475) (layers "F.Cu" "F.Paste" "F.Mask") (roundrect_rratio 0.25) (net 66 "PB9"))
  (pad "47" smd roundrect (at -2.25 -4.1625 90) (size 0.3 1.475) (layers "F.Cu" "F.Paste" "F.Mask") (roundrect_rratio 0.25) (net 2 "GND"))
  (pad "48" smd roundrect (at -2.75 -4.1625 90) (size 0.3 1.475) (layers "F.Cu" "F.Paste" "F.Mask") (roundrect_rratio 0.25) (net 1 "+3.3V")))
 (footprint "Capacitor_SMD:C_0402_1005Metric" (layer "F.Cu") (at 129.425 95.03 -90)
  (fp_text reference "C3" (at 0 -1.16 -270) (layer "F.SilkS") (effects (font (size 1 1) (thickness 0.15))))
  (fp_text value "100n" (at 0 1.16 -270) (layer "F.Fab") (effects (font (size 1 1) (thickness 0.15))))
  (pad "1" smd roundrect (at -0.48 0 270) (size 0.56 0.62) (layers "F.Cu" "F.Paste" "F.Mask") (roundrect_rratio 0.25) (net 1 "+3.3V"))
  (pad "2" smd roundrect (at 0.48 0 270) (size 0.56 0.62) (layers "F.Cu" "F.Paste" "F.Mask") (roundrect_rratio 0.25) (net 2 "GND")))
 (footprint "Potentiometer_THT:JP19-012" (layer "F.Cu") (at 156.18 92)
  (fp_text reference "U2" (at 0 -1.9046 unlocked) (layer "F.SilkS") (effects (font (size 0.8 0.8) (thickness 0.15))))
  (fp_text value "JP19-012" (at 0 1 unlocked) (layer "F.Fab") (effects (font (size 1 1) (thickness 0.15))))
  (pad "" thru_hole circle (at -8 0.65 90) (size 3.24 3.24) (drill 1.8) (layers "*.Cu" "*.Mask"))
  (pad "1" thru_hole rect (at 12.6 -8.6) (size 1.35 1.35) (drill 0.8) (layers "*.Cu" "*.Mask") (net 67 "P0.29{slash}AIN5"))
  (pad "2" thru_hole oval (at 12.6 -6.6) (size 1.35 1.35) (drill 0.8) (layers "*.Cu" "*.Mask") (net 2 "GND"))
  (pad "3" thru_hole oval (at 12.6 -4.6) (size 1.35 1.35) (drill 0.8) (layers "*.Cu" "*.Mask") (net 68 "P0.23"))
  (pad "4" thru_hole oval (at 12.6 -2.6) (size 1.35 1.35) (drill 0.8) (layers "*.Cu" "*.Mask") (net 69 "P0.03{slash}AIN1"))
  (pad "5" thru_hole oval (at 12.6 -0.6) (size 1.35 1.35) (drill 0.8) (layers "*.Cu" "*.Mask") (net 2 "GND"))
  (pad "6" thru_hole oval (at 12.6 1.4) (size 1.35 1.35) (drill 0.8) (layers "*.Cu" "*.Mask") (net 1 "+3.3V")))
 (gr_line (start 119.8025 103.13) (end 119.8025 65.13) (stroke (width 0.1) (type solid)) (layer "Edge.Cuts"))
 (gr_line (start 119.8025 65.13) (end 169.8025 65.13) (stroke (width 0.1) (type solid)) (layer "Edge.Cuts"))
 (gr_line (start 169.8025 103.13) (end 169.8025 65.13) (stroke (width 0.1) (type solid)) (layer "Edge.Cuts"))
 (gr_line (start 119.8025 103.13) (end 169.8025 103.13) (stroke (width 0.1) (type solid)) (layer "Edge.Cuts"))
 (segment (start 127.82 92.45) (end 127.55 92.72) (width 0.3) (layer "F.Cu") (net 2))
 (segment (start 133.97 94.3625) (end 133.97 95.7) (width 0.3) (layer "F.Cu") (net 2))
 (segment (start 130.97 86.0375) (end 130.97 84.67) (width 0.3) (layer "F.Cu") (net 2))
 (segment (start 137.3825 87.95) (end 138.73 87.95) (width 0.3) (layer "F.Cu") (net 2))
 (segment (start 129.075 98.96) (end 128.44 98.96) (width 0.5) (layer "F.Cu") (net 2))
 (segment (start 130.075 95.575) (end 129.49 95.575) (width 0.5) (layer "F.Cu") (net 2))
 (segment (start 129.0575 92.45) (end 127.82 92.45) (width 0.3) (layer "F.Cu") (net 2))
 (segment (start 129.49 95.575) (end 129.425 95.51) (width 0.5) (layer "F.Cu") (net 2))
 (segment (start 138.73 87.95) (end 138.9 87.78) (width 0.3) (layer "F.Cu") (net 2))
 (segment (start 128.44 98.96) (end 128.425 98.975) (width 0.5) (layer "F.Cu") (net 2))
 (segment (start 129.0575 92.45) (end 130.275 92.45) (width 0.3) (layer "F.Cu") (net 2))
 (segment (start 139.8 101.05) (end 140.675 101.05) (width 0.5) (layer "F.Cu") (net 2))
 (segment (start 125.3 89.85) (end 125.3 90.065) (width 0.5) (layer "F.Cu") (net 2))
 (segment (start 125.775 95.025) (end 126.575 95.025) (width 0.5) (layer "F.Cu") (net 2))
 (segment (start 133.745 95.925) (end 133.745 97.645) (width 0.5) (layer "F.Cu") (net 2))
 (segment (start 130.8 84.5) (end 130.8 83.79) (width 0.5) (layer "F.Cu") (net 2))
 (segment (start 133.97 95.7) (end 133.745 95.925) (width 0.3) (layer "F.Cu") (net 2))
 (segment (start 137.3825 87.95) (end 136.125 87.95) (width 0.3) (layer "F.Cu") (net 2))
 (segment (start 136.375 98.965) (end 137.015 98.965) (width 0.5) (layer "F.Cu") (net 2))
 (segment (start 130.97 84.67) (end 130.8 84.5) (width 0.3) (layer "F.Cu") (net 2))
 (segment (start 125.3 90.065) (end 125.675 90.44) (width 0.5) (layer "F.Cu") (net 2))
 (segment (start 133.97 94.3625) (end 133.97 93.13) (width 0.3) (layer "F.Cu") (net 2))
 (segment (start 133.745 97.645) (end 133.75 97.65) (width 0.5) (layer "F.Cu") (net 2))
 (segment (start 133.97 93.13) (end 133.975 93.125) (width 0.3) (layer "F.Cu") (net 2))
 (segment (start 137.015 98.965) (end 137.025 98.975) (width 0.5) (layer "F.Cu") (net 2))
 (via (at 130.275 92.45) (size 0.8) (drill 0.4) (layers "F.Cu" "B.Cu") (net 2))
 (via (at 137.025 98.975) (size 0.7) (drill 0.3) (layers "F.Cu" "B.Cu") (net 2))
 (via (at 130.075 95.575) (size 0.7) (drill 0.3) (layers "F.Cu" "B.Cu") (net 2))
 (via (at 140.675 101.05) (size 0.8) (drill 0.4) (layers "F.Cu" "B.Cu") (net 2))
 (via (at 133.75 97.65) (size 0.7) (drill 0.3) (layers "F.Cu" "B.Cu") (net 2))
 (via (at 133.975 93.125) (size 0.8) (drill 0.4) (layers "F.Cu" "B.Cu") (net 2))
 (via (at 125.775 95.025) (size 0.7) (drill 0.3) (layers "F.Cu" "B.Cu") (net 2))
 (via (at 136.125 87.95) (size 0.8) (drill 0.4) (layers "F.Cu" "B.Cu") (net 2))
 (via (at 128.425 98.975) (size 0.7) (drill 0.3) (layers "F.Cu" "B.Cu") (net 2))
 (via (at 125.3 89.85) (size 0.7) (drill 0.3) (layers "F.Cu" "B.Cu") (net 2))
 (via (at 130.8 83.79) (size 0.8) (drill 0.4) (layers "F.Cu" "B.Cu") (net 2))
 (segment (start 134.7 96.975) (end 134.7 95.93) (width 0.5) (layer "F.Cu") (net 9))
 (segment (start 134.7 95.93) (end 134.705 95.925) (width 0.5) (layer "F.Cu") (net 9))
 (segment (start 134.7 96.975) (end 135.7 96.975) (width 0.5) (layer "F.Cu") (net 9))
 (segment (start 134.47 95.69) (end 134.705 95.925) (width 0.3) (layer "F.Cu") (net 9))
 (segment (start 134.47 94.3625) (end 134.47 95.69) (width 0.3) (layer "F.Cu") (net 9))
 (segment (start 129.08 99.925) (end 129.075 99.92) (width 0.3) (layer "F.Cu") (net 4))
 (segment (start 132.47 94.3625) (end 132.47 96.93) (width 0.3) (layer "F.Cu") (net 4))
 (segment (start 130.875 98.525) (end 130.875 99.925) (width 0.3) (layer "F.Cu") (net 4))
 (segment (start 132.47 96.93) (end 130.875 98.525) (width 0.3) (layer "F.Cu") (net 4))
 (segment (start 130.875 99.925) (end 129.08 99.925) (width 0.3) (layer "F.Cu") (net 4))
 (segment (start 134.575 99.925) (end 136.375 99.925) (width 0.3) (layer "F.Cu") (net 7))
 (segment (start 132.97 98.32) (end 134.575 99.925) (width 0.3) (layer "F.Cu") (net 7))
 (segment (start 132.97 94.3625) (end 132.97 98.32) (width 0.3) (layer "F.Cu") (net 7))
 (segment (start 139.8 99.4) (end 139.8 97.8125) (width 0.5) (layer "F.Cu") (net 12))
 (segment (start 131.47 86.94) (end 131.11 87.3) (width 0.3) (layer "F.Cu") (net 31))
 (segment (start 131.11 87.3) (end 130.35 87.3) (width 0.3) (layer "F.Cu") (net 31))
 (segment (start 129.64 86.59) (end 129.64 85.83) (width 0.3) (layer "F.Cu") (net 31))
 (segment (start 131.47 86.0375) (end 131.47 86.94) (width 0.3) (layer "F.Cu") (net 31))
 (segment (start 130.35 87.3) (end 129.64 86.59) (width 0.3) (layer "F.Cu") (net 31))
 (segment (start 129.0575 92.95) (end 128.35 92.95) (width 0.3) (layer "F.Cu") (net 1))
 (segment (start 130.47 85.27) (end 129.84 84.64) (width 0.3) (layer "F.Cu") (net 1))
 (segment (start 129.6125 94.3625) (end 129.425 94.55) (width 0.3) (layer "F.Cu") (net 1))
 (segment (start 127.62 93.68) (end 127.55 93.68) (width 0.3) (layer "F.Cu") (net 1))
 (segment (start 128.125 95.025) (end 128.125 94.255) (width 0.5) (layer "F.Cu") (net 1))
 (segment (start 128.125 94.255) (end 127.55 93.68) (width 0.5) (layer "F.Cu") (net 1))
 (segment (start 128.6 94.55) (end 128.125 95.025) (width 0.5) (layer "F.Cu") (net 1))
 (segment (start 130.47 94.3625) (end 129.6125 94.3625) (width 0.3) (layer "F.Cu") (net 1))
 (segment (start 130.47 86.0375) (end 130.47 85.27) (width 0.3) (layer "F.Cu") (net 1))
 (segment (start 128.35 92.95) (end 127.62 93.68) (width 0.3) (layer "F.Cu") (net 1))
 (segment (start 138.78 86.82) (end 138.9 86.82) (width 0.3) (layer "F.Cu") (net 1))
 (segment (start 138.15 87.45) (end 138.78 86.82) (width 0.3) (layer "F.Cu") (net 1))
 (segment (start 137.3825 87.45) (end 138.15 87.45) (width 0.3) (layer "F.Cu") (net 1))
 (segment (start 129.425 94.55) (end 128.6 94.55) (width 0.5) (layer "F.Cu") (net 1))
 (segment (start 129.84 84.64) (end 129.84 84.5) (width 0.3) (layer "F.Cu") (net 1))
 (segment (start 126.185 90.95) (end 125.675 91.46) (width 0.3) (layer "F.Cu") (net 10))
 (segment (start 129.0575 90.95) (end 126.185 90.95) (width 0.3) (layer "F.Cu") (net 10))
 (segment (start 135.47 94.3625) (end 135.47 95.57) (width 0.3) (layer "F.Cu") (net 37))
 (segment (start 139.4625 95.9) (end 139.8 96.2375) (width 0.3) (layer "F.Cu") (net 37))
 (segment (start 135.8 95.9) (end 139.4625 95.9) (width 0.3) (layer "F.Cu") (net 37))
 (segment (start 135.47 95.57) (end 135.8 95.9) (width 0.3) (layer "F.Cu") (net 37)))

